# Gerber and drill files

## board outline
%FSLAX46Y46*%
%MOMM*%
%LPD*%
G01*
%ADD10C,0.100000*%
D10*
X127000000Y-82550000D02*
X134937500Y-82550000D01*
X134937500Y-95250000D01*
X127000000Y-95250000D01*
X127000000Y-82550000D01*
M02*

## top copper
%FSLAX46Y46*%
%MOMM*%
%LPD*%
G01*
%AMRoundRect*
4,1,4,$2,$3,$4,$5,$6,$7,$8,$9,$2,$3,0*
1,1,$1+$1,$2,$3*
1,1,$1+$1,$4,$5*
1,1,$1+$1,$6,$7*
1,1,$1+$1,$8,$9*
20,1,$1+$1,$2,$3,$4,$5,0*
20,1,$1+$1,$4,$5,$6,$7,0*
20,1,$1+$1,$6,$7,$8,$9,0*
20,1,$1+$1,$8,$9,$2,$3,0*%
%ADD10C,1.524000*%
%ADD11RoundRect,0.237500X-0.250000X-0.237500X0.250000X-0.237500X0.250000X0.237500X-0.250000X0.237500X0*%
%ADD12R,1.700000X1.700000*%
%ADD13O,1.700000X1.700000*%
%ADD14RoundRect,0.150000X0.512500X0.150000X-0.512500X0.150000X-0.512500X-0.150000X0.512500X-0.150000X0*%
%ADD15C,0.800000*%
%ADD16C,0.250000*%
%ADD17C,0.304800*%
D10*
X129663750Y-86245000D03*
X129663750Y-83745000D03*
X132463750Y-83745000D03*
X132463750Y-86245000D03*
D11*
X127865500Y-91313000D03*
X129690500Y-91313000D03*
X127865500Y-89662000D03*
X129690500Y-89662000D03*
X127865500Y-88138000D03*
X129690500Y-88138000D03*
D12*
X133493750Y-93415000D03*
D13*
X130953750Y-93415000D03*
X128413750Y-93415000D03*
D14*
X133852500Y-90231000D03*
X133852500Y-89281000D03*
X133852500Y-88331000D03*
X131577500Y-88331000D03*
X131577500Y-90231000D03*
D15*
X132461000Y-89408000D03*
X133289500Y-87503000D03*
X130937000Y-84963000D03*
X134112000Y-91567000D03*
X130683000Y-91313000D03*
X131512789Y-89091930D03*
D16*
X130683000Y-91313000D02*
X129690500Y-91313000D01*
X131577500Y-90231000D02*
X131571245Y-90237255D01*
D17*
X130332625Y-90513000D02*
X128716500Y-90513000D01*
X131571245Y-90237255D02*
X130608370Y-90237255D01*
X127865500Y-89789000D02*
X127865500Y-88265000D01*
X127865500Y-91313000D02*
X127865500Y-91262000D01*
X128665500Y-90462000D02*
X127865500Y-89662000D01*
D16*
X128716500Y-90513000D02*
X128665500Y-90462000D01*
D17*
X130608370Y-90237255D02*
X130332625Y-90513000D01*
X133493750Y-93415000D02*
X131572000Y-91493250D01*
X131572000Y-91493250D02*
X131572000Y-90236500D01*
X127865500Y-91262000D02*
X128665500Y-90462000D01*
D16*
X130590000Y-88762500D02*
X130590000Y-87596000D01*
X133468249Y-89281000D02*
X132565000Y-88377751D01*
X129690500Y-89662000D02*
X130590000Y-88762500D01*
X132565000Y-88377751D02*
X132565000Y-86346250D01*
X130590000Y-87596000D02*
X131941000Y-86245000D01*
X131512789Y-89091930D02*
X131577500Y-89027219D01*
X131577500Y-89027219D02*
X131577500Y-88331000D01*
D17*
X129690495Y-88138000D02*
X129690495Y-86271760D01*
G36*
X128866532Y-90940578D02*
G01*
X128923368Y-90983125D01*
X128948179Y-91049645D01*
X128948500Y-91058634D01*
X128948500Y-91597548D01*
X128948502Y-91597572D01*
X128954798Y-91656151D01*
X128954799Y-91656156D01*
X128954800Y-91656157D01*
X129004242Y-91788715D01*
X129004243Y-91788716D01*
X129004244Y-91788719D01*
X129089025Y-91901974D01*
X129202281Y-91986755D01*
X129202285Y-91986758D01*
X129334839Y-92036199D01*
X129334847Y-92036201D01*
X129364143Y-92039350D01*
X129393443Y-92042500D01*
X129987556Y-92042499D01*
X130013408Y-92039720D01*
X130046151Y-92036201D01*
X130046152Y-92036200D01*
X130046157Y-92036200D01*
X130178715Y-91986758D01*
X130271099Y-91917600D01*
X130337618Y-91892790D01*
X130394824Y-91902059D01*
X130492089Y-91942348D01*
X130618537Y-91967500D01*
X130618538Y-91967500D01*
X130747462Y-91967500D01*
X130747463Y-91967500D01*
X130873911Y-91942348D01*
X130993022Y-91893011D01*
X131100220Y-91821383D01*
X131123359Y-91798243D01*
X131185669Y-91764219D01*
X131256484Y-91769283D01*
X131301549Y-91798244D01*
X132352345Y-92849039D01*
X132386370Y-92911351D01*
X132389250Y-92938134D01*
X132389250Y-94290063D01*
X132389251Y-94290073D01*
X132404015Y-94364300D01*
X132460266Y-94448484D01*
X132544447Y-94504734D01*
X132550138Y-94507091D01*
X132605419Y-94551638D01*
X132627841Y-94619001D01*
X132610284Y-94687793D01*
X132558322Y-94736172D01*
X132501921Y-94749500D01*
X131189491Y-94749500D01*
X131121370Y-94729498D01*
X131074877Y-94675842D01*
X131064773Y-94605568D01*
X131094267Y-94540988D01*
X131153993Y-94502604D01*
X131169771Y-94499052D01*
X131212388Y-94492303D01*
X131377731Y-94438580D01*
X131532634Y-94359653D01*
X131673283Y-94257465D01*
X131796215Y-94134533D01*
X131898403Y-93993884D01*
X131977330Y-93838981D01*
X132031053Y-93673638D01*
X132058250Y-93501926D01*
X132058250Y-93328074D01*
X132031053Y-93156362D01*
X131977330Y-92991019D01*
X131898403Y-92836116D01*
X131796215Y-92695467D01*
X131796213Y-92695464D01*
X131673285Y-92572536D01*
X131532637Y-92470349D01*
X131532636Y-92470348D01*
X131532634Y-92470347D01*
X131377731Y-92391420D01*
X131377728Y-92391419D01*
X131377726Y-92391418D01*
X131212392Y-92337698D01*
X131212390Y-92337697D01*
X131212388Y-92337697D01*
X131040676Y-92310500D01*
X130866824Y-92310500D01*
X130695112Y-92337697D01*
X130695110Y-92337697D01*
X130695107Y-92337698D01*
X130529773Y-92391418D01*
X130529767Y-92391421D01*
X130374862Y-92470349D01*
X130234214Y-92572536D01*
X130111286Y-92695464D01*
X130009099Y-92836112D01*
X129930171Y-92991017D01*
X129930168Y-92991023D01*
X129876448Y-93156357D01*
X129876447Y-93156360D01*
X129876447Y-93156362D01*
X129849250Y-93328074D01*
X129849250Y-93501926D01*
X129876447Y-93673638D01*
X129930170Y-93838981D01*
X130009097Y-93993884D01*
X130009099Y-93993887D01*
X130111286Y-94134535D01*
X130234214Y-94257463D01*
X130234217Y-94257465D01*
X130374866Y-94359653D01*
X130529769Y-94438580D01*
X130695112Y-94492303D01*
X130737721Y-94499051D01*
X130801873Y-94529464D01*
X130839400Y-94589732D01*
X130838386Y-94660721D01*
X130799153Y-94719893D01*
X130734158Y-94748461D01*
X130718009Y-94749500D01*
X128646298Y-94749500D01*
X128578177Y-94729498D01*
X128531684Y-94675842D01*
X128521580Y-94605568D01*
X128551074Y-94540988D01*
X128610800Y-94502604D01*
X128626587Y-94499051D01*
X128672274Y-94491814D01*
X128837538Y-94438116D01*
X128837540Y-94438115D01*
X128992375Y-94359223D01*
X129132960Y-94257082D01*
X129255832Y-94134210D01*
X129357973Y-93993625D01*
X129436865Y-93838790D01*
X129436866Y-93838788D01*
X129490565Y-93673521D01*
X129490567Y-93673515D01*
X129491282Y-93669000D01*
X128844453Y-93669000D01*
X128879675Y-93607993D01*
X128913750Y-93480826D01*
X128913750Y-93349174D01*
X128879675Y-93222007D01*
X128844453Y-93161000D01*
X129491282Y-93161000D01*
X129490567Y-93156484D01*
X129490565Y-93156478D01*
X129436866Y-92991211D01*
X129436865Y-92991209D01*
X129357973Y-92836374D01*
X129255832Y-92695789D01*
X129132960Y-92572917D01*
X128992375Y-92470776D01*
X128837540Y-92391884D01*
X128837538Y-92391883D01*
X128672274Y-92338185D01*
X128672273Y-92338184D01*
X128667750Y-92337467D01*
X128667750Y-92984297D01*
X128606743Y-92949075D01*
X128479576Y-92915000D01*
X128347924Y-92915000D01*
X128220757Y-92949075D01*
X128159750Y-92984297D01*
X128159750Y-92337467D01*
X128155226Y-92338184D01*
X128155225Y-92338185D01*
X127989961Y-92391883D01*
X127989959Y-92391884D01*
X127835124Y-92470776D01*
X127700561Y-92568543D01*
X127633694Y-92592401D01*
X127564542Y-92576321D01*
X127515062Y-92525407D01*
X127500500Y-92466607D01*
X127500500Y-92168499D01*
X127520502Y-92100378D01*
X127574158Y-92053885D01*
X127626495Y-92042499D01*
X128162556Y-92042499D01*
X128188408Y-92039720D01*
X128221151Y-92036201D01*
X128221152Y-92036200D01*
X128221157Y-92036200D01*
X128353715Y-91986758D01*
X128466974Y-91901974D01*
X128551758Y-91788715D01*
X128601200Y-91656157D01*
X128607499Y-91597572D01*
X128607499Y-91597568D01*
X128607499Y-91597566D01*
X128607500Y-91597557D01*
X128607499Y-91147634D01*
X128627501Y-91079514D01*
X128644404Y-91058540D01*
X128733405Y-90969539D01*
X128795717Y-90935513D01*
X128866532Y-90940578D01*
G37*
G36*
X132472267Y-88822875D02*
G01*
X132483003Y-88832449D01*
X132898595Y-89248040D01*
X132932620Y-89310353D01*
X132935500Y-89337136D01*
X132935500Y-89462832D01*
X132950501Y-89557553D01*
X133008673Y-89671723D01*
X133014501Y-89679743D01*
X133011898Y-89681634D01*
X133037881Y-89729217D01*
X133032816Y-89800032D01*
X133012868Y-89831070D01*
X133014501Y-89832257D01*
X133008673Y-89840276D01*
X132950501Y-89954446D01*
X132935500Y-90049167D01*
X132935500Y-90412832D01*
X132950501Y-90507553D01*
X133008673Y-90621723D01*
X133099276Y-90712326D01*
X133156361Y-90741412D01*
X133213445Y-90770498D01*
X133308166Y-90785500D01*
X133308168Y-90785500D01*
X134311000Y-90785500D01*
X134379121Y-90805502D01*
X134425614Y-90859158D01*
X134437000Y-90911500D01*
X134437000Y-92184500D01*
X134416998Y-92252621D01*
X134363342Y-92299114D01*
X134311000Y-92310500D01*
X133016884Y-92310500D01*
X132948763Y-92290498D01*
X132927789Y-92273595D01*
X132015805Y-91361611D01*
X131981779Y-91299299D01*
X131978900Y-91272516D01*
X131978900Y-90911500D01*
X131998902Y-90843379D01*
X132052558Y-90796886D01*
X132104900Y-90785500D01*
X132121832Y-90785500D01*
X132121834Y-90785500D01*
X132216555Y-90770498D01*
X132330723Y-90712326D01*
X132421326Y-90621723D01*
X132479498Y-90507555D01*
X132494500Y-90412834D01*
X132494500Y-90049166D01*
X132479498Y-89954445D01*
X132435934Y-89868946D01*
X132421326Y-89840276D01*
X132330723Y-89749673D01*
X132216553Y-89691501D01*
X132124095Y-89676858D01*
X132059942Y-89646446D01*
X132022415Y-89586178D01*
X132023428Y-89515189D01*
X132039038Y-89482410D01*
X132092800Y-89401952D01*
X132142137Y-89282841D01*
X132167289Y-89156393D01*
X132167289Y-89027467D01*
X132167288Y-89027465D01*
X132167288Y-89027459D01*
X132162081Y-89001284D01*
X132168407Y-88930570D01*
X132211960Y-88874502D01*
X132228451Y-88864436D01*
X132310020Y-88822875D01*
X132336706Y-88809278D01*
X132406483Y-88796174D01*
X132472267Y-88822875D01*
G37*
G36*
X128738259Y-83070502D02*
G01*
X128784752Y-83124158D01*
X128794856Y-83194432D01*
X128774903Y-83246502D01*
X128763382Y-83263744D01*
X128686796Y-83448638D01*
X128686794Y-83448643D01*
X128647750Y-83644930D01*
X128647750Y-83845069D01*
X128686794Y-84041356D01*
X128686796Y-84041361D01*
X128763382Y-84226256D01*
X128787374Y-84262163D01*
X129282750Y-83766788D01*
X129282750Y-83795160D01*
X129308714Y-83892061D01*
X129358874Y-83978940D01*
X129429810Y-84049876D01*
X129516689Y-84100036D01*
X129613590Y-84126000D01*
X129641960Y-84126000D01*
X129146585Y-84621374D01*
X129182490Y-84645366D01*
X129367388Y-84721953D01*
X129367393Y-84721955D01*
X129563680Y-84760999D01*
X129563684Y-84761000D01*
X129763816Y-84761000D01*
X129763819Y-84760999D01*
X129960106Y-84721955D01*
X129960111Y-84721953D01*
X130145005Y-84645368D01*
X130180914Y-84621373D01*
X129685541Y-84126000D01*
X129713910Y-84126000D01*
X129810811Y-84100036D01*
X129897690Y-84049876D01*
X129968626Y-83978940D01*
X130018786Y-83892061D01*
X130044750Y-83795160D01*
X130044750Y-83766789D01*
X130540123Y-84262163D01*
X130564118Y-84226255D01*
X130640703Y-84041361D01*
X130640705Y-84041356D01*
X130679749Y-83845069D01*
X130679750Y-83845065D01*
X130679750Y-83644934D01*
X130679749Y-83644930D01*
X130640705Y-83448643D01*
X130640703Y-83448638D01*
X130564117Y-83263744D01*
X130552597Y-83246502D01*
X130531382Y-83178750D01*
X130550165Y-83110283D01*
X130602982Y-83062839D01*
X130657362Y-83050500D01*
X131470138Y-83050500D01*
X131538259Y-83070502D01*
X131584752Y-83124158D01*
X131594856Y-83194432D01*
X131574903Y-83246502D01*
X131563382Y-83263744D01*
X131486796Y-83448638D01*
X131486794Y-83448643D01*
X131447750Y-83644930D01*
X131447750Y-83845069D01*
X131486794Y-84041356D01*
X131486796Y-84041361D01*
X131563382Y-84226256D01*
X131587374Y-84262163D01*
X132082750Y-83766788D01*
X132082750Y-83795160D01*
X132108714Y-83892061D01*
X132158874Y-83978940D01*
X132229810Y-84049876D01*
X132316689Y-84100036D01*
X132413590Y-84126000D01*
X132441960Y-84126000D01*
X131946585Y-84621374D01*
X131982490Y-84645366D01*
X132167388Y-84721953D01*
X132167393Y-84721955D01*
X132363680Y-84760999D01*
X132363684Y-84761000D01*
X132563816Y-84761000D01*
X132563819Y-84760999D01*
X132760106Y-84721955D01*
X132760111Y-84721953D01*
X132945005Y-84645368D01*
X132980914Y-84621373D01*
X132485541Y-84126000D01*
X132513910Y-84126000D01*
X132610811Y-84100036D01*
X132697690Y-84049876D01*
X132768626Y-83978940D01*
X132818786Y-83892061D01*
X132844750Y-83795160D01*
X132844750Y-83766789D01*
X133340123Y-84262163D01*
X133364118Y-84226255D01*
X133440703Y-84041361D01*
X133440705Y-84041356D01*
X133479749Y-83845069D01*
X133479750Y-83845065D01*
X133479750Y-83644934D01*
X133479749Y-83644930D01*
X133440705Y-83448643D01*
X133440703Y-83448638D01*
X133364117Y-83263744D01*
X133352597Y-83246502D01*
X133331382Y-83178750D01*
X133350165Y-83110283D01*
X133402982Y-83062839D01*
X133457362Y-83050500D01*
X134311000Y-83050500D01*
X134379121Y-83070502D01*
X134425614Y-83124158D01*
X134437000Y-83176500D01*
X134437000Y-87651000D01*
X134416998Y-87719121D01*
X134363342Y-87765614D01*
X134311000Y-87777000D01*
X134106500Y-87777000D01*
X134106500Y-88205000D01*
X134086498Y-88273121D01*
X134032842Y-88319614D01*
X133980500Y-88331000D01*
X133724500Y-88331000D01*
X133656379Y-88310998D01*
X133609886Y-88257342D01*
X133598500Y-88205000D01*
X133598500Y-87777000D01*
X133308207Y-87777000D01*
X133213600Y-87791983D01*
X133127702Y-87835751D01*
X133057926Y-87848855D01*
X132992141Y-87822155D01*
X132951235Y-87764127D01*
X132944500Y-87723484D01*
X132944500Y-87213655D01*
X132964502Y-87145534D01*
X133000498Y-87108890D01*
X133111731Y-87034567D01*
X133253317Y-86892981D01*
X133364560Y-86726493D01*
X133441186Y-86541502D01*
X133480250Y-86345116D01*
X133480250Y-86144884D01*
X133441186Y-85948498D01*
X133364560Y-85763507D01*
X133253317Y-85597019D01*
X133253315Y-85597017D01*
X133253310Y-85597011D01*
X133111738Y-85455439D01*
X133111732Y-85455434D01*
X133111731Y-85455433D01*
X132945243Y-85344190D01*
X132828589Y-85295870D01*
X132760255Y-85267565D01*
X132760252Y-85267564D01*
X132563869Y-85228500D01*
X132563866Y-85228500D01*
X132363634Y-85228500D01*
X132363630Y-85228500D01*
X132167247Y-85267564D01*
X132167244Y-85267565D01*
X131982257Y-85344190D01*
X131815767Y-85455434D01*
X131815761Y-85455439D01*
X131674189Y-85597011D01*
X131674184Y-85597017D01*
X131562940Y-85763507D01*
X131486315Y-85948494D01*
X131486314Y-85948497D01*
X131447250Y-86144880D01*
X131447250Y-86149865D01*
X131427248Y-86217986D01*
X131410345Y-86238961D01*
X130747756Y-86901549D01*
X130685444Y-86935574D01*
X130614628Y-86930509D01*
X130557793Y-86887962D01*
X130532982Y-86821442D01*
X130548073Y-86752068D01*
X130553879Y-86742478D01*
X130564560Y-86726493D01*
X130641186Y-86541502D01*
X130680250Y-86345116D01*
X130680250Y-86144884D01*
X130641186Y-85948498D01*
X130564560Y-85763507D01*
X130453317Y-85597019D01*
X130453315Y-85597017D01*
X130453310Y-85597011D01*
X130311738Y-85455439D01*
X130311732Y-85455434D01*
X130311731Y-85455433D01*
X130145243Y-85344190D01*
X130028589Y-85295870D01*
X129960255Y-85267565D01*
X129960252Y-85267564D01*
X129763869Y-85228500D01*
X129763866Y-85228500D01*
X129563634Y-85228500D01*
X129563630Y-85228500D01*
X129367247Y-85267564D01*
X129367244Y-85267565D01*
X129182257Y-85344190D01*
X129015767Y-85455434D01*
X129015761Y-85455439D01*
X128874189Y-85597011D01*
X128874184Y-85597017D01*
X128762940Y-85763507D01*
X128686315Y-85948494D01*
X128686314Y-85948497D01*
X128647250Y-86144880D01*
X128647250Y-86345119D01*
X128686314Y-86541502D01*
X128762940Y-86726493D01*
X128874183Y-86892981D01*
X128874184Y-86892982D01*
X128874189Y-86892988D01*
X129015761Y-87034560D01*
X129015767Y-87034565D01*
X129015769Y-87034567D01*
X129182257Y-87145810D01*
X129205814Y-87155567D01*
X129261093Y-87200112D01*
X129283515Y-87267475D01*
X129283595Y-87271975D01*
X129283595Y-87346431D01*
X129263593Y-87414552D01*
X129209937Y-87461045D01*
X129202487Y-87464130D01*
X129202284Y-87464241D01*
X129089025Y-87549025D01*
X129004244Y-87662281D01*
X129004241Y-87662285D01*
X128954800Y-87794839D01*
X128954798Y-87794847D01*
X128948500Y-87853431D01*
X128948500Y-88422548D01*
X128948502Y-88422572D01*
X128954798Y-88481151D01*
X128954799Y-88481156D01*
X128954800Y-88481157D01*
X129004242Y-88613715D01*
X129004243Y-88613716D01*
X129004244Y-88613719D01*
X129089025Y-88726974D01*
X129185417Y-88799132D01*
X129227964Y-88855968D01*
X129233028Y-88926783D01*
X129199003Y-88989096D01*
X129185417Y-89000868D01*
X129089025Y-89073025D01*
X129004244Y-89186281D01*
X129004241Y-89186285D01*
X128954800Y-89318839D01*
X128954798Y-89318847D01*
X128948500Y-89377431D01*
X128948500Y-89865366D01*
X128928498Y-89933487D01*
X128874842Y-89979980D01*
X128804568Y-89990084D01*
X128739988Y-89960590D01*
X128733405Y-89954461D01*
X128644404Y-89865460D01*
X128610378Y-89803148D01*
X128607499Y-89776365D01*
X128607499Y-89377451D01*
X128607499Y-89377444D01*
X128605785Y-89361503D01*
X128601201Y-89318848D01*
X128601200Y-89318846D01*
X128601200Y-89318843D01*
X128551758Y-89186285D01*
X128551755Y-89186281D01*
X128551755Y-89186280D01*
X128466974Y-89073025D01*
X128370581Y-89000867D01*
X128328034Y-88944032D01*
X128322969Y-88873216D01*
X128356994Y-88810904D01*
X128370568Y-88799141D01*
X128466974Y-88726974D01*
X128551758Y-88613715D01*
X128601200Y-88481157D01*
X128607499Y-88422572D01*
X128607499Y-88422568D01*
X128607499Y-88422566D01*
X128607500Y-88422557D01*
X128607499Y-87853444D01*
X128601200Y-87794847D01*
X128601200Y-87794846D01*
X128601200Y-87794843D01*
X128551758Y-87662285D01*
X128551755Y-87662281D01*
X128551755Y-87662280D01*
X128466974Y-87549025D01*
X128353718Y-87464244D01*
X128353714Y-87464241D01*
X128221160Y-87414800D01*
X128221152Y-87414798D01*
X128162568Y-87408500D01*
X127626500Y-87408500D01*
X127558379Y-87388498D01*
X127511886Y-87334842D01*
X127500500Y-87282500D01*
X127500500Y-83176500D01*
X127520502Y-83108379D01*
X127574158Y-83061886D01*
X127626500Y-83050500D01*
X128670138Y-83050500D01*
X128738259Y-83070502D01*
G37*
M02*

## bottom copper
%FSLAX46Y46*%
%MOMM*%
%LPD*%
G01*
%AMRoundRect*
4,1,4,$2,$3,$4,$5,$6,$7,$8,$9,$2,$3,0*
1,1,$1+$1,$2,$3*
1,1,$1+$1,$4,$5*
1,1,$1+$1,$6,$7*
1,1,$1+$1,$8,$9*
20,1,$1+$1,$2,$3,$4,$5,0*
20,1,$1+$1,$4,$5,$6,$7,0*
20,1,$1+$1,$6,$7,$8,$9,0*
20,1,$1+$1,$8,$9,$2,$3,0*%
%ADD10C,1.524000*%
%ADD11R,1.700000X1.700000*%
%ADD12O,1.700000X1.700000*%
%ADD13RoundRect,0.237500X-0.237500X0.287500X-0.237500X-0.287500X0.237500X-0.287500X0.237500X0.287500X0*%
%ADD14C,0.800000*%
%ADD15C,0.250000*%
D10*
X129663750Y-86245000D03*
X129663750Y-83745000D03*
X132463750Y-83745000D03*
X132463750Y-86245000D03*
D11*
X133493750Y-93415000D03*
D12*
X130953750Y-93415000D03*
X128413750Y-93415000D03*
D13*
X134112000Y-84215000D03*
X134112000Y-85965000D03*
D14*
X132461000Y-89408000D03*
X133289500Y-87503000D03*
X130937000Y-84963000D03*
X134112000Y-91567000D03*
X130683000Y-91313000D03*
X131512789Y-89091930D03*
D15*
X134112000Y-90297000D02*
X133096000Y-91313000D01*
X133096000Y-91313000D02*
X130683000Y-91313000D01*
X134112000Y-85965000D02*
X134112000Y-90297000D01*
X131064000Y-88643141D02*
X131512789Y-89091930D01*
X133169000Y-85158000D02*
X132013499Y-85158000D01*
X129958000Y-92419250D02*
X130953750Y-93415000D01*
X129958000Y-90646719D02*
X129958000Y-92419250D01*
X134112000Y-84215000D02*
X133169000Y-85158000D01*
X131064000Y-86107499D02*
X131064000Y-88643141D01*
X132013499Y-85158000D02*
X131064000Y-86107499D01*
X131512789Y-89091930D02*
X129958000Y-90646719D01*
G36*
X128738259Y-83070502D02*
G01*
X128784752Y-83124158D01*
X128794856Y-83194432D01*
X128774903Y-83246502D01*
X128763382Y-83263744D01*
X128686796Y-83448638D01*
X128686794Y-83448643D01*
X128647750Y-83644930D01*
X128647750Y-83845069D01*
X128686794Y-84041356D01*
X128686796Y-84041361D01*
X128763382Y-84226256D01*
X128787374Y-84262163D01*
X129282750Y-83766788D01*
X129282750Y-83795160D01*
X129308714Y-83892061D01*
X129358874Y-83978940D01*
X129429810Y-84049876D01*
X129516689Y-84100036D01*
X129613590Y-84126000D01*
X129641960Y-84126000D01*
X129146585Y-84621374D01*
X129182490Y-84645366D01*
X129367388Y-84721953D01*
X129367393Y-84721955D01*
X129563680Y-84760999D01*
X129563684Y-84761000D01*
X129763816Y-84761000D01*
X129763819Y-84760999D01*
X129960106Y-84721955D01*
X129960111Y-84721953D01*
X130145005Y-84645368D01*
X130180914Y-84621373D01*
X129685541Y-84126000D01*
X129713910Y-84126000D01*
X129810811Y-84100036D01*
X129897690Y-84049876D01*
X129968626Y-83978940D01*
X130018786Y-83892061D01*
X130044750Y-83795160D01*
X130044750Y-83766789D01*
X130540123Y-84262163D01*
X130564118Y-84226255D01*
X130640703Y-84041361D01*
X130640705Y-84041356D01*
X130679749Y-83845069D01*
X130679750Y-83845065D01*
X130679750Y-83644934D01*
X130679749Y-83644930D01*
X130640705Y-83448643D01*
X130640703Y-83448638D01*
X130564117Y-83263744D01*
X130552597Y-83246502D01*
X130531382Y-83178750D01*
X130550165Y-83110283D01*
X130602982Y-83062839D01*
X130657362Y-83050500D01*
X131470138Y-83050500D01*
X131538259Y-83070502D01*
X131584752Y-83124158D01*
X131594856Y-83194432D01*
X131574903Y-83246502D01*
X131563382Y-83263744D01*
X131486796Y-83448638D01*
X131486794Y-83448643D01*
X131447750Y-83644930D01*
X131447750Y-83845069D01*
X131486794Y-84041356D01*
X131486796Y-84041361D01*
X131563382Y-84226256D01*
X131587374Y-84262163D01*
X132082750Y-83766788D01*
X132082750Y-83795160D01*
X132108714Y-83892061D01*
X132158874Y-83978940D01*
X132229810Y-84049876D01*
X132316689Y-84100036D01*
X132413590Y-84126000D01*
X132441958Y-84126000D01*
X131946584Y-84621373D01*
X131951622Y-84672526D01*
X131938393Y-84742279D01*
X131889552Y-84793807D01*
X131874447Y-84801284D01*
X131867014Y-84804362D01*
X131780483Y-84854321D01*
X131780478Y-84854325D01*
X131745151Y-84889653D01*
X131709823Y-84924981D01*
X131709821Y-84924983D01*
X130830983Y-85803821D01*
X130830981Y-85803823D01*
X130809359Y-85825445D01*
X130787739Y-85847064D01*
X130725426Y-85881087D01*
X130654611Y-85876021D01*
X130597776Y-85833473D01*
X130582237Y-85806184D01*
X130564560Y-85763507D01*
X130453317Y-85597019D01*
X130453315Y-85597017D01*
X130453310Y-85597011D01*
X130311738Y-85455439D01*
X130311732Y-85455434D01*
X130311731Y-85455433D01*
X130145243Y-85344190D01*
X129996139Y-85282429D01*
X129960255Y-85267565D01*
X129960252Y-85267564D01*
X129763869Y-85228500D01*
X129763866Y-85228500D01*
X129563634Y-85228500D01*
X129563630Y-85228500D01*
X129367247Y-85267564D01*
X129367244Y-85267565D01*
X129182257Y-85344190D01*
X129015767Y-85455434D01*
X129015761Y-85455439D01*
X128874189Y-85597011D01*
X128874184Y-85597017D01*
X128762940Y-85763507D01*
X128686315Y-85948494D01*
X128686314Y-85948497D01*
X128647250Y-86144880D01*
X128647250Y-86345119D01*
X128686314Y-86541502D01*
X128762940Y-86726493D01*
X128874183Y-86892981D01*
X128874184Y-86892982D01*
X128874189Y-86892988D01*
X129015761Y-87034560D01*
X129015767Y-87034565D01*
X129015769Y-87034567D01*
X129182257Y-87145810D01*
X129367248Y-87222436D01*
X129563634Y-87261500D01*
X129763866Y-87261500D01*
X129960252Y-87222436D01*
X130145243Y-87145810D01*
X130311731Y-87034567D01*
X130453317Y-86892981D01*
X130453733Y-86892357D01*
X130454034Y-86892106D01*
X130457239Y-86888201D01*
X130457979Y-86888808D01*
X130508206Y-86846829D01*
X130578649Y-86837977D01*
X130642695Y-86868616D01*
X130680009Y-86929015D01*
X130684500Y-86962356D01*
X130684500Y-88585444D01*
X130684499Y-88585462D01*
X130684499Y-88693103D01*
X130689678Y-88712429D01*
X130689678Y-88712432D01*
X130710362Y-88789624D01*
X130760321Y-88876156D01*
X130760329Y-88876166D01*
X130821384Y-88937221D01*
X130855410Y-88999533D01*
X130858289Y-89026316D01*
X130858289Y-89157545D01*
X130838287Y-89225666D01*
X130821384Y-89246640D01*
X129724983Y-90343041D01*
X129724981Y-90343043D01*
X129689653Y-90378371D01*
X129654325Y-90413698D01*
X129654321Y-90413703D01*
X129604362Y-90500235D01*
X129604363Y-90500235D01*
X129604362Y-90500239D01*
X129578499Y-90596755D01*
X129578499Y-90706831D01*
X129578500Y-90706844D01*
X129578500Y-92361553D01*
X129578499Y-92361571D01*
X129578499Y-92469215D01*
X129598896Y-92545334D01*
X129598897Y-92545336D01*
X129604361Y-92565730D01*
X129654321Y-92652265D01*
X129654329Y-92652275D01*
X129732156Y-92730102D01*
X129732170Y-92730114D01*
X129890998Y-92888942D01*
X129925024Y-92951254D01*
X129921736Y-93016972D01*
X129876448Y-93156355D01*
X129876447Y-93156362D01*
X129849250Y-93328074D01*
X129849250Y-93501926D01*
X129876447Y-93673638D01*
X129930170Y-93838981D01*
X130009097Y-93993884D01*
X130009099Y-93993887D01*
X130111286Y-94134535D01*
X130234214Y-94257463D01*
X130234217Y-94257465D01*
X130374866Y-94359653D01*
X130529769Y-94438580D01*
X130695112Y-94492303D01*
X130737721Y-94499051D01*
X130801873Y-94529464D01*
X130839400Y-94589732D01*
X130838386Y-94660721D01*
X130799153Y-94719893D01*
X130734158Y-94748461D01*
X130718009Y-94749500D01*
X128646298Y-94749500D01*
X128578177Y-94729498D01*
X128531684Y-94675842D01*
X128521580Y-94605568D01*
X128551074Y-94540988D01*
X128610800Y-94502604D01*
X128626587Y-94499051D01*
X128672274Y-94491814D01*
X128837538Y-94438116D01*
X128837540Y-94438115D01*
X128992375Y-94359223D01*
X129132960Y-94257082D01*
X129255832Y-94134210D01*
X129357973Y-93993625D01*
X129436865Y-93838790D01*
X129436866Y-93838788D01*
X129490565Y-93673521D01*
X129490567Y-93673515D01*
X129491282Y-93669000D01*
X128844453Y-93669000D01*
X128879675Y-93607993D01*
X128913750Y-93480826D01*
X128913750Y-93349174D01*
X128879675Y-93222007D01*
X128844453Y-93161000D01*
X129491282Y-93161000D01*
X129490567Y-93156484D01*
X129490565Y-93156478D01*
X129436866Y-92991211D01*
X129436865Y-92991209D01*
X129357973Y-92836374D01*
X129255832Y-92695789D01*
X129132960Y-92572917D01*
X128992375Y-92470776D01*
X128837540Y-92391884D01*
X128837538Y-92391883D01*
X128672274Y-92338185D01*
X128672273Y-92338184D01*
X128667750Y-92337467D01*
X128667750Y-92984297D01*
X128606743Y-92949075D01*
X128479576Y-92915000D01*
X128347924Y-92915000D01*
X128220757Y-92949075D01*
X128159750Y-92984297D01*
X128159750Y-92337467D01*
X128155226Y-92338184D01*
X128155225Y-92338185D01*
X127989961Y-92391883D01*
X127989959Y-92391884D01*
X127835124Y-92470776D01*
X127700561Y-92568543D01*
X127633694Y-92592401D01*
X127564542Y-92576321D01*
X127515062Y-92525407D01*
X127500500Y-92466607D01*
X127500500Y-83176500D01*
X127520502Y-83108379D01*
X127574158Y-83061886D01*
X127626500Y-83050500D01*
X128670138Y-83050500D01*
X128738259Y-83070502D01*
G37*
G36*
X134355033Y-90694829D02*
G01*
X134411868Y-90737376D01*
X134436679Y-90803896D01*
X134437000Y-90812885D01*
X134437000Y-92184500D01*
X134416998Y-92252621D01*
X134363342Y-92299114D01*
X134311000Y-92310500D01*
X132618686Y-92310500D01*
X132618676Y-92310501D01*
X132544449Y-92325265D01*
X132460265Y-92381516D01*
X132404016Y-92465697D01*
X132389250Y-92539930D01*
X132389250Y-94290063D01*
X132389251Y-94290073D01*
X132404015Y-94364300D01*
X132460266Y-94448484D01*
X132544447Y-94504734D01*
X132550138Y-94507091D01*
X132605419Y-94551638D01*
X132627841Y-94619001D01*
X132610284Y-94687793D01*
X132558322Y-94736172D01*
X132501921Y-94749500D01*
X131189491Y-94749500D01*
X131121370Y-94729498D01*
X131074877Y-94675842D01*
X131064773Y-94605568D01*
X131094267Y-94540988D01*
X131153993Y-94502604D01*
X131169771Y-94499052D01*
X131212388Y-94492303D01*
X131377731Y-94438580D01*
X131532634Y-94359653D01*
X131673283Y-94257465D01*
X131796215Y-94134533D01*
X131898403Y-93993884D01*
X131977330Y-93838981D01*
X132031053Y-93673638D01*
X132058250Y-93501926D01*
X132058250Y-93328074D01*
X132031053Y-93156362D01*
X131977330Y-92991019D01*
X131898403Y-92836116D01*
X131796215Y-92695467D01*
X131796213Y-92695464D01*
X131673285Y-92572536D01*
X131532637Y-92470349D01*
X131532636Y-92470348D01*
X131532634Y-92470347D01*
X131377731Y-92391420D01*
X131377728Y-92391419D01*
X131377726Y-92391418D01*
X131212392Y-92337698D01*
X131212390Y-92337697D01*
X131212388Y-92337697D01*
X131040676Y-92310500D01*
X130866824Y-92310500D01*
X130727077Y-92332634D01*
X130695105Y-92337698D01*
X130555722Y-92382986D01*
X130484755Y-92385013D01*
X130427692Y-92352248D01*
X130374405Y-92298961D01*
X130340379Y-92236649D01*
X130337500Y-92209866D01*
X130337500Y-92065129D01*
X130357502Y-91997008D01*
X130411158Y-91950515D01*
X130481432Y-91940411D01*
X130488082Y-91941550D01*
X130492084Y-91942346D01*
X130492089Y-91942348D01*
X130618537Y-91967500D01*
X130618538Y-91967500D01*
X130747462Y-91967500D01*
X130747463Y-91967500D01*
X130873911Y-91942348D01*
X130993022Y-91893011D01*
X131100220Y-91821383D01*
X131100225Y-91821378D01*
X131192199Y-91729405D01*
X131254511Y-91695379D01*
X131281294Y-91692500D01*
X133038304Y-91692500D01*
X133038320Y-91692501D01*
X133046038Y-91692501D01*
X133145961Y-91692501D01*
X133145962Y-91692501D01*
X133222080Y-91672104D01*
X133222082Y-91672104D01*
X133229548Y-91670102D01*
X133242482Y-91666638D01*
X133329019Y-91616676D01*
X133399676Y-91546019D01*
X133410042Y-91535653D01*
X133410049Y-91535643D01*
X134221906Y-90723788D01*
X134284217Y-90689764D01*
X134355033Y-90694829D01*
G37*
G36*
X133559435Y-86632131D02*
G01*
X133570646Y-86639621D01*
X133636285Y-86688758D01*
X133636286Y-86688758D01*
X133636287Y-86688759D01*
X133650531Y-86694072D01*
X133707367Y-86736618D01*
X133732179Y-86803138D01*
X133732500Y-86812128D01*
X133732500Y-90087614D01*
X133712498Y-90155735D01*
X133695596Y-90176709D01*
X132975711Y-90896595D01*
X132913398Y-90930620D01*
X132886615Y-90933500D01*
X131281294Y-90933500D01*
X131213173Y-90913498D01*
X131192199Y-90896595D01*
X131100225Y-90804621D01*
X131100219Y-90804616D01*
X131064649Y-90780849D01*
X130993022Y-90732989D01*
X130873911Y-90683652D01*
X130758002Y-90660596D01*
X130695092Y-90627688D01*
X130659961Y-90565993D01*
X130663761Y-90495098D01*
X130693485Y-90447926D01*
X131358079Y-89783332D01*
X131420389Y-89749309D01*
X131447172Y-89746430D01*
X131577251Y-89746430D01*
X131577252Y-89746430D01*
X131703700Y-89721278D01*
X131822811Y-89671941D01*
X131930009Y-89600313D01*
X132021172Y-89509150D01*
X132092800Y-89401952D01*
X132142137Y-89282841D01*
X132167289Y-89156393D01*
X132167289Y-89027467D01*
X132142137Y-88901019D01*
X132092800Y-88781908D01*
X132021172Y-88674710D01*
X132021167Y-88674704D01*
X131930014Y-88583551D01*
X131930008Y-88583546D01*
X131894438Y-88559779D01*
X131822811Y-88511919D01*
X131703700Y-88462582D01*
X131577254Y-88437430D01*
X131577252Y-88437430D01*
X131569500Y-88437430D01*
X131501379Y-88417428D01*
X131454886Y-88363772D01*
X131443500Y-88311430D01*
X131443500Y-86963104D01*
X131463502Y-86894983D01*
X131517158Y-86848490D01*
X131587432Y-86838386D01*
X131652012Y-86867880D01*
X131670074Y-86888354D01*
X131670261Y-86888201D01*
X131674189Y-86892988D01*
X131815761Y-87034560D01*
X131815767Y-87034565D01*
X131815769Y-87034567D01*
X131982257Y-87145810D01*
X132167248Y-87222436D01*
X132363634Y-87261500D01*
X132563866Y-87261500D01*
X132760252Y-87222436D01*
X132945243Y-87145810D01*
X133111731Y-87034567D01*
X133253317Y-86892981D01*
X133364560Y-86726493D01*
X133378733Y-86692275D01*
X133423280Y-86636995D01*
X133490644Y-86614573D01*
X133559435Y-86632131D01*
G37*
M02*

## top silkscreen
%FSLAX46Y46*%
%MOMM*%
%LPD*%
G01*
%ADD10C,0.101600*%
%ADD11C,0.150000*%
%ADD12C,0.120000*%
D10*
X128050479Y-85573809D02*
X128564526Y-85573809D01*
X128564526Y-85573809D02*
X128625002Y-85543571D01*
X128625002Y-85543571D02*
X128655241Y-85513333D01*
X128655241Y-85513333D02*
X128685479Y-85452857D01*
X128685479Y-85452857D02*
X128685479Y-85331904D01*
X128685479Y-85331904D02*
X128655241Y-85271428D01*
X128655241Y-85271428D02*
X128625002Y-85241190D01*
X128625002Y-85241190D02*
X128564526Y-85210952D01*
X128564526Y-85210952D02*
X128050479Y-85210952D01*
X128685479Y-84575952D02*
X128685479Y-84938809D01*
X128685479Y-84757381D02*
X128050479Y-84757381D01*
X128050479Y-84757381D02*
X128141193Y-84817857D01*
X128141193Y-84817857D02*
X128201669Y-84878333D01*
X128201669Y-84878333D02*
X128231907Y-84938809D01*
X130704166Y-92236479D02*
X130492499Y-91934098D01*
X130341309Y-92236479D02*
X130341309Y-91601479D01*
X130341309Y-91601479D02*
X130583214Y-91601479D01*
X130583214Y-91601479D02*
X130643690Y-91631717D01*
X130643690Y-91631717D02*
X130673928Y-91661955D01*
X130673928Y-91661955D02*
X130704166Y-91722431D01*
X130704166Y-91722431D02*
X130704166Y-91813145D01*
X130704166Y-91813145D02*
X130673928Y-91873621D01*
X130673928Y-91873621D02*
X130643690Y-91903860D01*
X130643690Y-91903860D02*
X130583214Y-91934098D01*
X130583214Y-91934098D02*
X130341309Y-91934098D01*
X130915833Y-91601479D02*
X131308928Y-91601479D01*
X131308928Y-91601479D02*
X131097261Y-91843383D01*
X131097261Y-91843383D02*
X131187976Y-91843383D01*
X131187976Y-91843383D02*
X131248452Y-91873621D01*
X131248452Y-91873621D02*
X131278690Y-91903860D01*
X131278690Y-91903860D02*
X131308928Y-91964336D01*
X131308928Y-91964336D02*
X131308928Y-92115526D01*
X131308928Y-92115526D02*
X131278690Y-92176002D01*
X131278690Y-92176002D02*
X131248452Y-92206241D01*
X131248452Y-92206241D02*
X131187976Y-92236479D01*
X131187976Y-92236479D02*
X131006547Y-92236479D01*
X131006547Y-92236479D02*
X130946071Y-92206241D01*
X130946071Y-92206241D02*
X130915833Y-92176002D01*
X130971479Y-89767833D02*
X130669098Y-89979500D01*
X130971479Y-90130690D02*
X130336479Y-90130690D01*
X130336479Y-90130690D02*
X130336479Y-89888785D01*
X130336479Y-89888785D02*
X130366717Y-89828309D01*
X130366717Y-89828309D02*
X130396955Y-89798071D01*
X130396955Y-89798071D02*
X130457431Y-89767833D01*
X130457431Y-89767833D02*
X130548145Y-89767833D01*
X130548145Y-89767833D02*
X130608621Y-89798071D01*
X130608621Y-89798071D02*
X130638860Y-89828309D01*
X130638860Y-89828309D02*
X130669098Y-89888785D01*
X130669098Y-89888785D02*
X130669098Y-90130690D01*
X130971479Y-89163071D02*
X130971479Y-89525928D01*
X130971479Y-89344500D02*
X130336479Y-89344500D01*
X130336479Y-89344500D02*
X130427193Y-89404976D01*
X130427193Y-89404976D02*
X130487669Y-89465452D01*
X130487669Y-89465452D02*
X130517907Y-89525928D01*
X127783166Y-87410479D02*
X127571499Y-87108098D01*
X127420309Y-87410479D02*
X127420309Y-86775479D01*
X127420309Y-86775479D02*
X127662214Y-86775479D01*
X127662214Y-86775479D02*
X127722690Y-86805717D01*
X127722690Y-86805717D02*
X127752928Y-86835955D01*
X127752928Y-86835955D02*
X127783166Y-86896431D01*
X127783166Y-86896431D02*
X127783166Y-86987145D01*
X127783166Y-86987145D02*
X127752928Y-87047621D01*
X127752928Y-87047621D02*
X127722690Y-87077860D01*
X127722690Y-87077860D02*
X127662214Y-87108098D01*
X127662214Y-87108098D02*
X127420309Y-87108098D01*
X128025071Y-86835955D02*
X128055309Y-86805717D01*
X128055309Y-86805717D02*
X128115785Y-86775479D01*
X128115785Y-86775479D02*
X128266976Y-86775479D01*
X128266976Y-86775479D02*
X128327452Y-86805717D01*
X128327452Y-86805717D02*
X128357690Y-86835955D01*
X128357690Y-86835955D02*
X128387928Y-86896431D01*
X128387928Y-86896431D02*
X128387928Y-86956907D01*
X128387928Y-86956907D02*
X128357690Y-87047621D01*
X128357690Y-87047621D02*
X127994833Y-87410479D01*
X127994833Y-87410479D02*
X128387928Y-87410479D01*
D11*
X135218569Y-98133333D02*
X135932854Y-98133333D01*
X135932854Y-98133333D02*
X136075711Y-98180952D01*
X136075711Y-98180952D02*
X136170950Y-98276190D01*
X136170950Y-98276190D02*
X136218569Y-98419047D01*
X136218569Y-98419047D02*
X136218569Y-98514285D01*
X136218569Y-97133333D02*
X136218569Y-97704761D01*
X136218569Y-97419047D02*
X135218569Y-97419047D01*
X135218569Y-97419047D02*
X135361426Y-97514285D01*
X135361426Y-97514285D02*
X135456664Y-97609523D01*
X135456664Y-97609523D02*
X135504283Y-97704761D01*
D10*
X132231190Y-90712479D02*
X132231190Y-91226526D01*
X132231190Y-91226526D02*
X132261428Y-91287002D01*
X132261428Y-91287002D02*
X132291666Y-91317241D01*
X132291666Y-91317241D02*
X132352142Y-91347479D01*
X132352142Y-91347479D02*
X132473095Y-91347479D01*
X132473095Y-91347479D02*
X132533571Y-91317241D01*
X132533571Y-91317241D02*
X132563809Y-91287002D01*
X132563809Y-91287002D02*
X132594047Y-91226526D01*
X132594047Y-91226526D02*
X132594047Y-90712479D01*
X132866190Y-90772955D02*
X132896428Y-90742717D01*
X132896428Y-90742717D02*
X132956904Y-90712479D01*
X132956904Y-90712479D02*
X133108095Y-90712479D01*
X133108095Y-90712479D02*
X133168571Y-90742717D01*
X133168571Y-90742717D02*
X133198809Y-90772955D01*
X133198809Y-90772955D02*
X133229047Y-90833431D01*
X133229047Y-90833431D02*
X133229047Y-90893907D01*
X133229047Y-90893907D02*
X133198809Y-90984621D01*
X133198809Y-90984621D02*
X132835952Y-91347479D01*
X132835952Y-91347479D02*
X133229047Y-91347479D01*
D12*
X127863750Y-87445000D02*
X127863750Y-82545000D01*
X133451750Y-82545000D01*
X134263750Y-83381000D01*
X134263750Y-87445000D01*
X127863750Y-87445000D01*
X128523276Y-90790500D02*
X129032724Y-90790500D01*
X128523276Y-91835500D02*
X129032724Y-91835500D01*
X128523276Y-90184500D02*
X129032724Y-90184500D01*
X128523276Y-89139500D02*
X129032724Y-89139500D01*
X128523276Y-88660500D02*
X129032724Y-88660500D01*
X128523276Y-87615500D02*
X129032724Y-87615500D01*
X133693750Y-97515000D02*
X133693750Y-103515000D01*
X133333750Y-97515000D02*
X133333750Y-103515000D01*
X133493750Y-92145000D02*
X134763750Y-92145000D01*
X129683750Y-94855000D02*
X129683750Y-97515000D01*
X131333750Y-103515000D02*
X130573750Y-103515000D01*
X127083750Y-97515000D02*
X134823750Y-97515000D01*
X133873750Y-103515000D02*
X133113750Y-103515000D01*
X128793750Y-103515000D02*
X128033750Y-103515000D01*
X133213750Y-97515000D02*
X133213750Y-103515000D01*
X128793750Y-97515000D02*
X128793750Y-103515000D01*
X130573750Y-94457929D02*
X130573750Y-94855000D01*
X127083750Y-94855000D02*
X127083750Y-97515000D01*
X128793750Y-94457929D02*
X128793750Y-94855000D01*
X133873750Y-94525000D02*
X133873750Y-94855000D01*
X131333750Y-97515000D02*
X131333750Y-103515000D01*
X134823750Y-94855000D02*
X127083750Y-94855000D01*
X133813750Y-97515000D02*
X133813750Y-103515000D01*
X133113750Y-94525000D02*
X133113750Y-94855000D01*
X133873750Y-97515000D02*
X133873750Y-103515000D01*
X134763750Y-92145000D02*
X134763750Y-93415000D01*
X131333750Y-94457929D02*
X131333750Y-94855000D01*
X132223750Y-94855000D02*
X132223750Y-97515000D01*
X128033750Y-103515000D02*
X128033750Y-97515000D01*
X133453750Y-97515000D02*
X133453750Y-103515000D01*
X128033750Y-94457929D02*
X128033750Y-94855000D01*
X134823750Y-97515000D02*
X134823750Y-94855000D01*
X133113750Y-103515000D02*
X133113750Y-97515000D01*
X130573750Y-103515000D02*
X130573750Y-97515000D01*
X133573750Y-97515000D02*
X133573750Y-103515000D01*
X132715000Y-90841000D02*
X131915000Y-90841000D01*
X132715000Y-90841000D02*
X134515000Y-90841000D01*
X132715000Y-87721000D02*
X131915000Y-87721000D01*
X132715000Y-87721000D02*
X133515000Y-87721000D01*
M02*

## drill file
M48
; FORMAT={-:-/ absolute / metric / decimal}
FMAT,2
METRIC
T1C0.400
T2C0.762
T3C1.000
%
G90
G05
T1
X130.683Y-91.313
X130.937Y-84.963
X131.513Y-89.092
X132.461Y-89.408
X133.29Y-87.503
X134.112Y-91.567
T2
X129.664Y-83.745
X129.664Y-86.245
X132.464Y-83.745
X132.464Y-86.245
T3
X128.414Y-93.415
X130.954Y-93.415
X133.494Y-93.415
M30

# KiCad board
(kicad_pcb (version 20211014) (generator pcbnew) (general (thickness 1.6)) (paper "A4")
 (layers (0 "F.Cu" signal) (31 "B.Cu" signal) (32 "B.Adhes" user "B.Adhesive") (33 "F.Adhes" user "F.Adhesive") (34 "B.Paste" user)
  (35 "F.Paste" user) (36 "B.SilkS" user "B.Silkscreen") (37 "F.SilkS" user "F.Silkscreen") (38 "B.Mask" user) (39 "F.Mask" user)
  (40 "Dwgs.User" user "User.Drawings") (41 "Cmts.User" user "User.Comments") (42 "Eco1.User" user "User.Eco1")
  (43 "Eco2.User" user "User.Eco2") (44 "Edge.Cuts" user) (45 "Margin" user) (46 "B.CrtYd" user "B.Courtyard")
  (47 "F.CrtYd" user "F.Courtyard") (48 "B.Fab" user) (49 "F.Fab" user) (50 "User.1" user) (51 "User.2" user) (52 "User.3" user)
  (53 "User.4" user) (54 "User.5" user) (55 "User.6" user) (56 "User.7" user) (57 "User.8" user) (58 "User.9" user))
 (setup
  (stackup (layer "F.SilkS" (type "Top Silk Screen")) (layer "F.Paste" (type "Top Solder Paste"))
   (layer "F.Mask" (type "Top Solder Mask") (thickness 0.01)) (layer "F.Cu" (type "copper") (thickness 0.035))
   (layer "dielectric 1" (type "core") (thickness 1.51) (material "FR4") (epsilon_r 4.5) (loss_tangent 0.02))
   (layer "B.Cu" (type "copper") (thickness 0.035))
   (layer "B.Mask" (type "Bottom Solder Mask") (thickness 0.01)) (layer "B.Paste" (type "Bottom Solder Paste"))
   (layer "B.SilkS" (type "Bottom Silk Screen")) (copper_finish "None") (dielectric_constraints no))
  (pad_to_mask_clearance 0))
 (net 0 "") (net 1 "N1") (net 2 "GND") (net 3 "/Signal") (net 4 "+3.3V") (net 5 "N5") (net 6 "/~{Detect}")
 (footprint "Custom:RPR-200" (layer "F.Cu") (at 127.86375 87.445)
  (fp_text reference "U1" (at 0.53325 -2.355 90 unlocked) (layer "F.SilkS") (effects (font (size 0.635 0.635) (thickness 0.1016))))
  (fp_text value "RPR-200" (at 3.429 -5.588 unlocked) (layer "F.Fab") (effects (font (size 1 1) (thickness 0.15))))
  (fp_poly (pts (xy 0 0) (xy 0 -4.9) (xy 5.588 -4.9) (xy 6.4 -4.064) (xy 6.4 0)) (layer "F.SilkS") (width 0.12) (fill none))
  (pad "1" thru_hole circle (at 1.8 -1.2) (size 1.524 1.524) (drill 0.762) (layers *.Cu *.Mask) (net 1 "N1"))
  (pad "2" thru_hole circle (at 1.8 -3.7) (size 1.524 1.524) (drill 0.762) (layers *.Cu *.Mask) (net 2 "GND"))
  (pad "3" thru_hole circle (at 4.6 -3.7) (size 1.524 1.524) (drill 0.762) (layers *.Cu *.Mask) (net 2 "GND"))
  (pad "4" thru_hole circle (at 4.6 -1.2) (size 1.524 1.524) (drill 0.762) (layers *.Cu *.Mask) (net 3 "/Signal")))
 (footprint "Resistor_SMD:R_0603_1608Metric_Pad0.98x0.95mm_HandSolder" (layer "F.Cu") (at 128.778 91.313)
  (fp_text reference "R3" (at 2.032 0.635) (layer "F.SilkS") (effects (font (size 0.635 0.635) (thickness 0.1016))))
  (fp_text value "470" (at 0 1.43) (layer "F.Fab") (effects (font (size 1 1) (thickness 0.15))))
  (fp_line (start -0.254724 -0.5225) (end 0.254724 -0.5225) (layer "F.SilkS") (width 0.12))
  (fp_line (start -0.254724 0.5225) (end 0.254724 0.5225) (layer "F.SilkS") (width 0.12))
  (pad "1" smd roundrect (at -0.9125 0) (size 0.975 0.95) (layers "F.Cu" "F.Paste" "F.Mask") (roundrect_rratio 0.25) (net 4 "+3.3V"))
  (pad "2" smd roundrect (at 0.9125 0) (size 0.975 0.95) (layers "F.Cu" "F.Paste" "F.Mask") (roundrect_rratio 0.25) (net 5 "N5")))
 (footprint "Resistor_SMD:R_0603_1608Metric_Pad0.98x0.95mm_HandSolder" (layer "F.Cu") (at 128.778 89.662)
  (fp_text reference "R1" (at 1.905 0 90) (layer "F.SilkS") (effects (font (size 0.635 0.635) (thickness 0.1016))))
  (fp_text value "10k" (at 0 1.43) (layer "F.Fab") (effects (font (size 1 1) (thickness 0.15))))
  (fp_line (start -0.254724 0.5225) (end 0.254724 0.5225) (layer "F.SilkS") (width 0.12))
  (fp_line (start -0.254724 -0.5225) (end 0.254724 -0.5225) (layer "F.SilkS") (width 0.12))
  (pad "1" smd roundrect (at -0.9125 0) (size 0.975 0.95) (layers "F.Cu" "F.Paste" "F.Mask") (roundrect_rratio 0.25) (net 4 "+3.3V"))
  (pad "2" smd roundrect (at 0.9125 0) (size 0.975 0.95) (layers "F.Cu" "F.Paste" "F.Mask") (roundrect_rratio 0.25) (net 3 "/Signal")))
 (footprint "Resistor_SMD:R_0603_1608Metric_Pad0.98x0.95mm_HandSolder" (layer "F.Cu") (at 128.778 88.138)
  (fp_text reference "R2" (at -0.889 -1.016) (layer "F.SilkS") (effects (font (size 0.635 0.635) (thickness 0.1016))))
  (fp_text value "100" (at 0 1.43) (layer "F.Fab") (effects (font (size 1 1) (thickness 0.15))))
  (fp_line (start -0.254724 0.5225) (end 0.254724 0.5225) (layer "F.SilkS") (width 0.12))
  (fp_line (start -0.254724 -0.5225) (end 0.254724 -0.5225) (layer "F.SilkS") (width 0.12))
  (pad "1" smd roundrect (at -0.9125 0) (size 0.975 0.95) (layers "F.Cu" "F.Paste" "F.Mask") (roundrect_rratio 0.25) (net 4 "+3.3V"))
  (pad "2" smd roundrect (at 0.9125 0) (size 0.975 0.95) (layers "F.Cu" "F.Paste" "F.Mask") (roundrect_rratio 0.25) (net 1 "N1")))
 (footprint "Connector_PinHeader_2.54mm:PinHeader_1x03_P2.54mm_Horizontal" (layer "F.Cu") (at 133.49375 93.415 -90)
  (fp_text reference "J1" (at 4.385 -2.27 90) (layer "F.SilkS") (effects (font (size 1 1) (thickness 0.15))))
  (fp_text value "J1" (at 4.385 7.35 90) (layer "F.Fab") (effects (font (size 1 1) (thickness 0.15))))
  (fp_line (start 4.1 -0.2) (end 10.1 -0.2) (layer "F.SilkS") (width 0.12))
  (fp_line (start 4.1 0.16) (end 10.1 0.16) (layer "F.SilkS") (width 0.12))
  (fp_line (start -1.27 0) (end -1.27 -1.27) (layer "F.SilkS") (width 0.12))
  (fp_line (start 1.44 3.81) (end 4.1 3.81) (layer "F.SilkS") (width 0.12))
  (fp_line (start 10.1 2.16) (end 10.1 2.92) (layer "F.SilkS") (width 0.12))
  (fp_line (start 4.1 6.41) (end 4.1 -1.33) (layer "F.SilkS") (width 0.12))
  (fp_line (start 10.1 -0.38) (end 10.1 0.38) (layer "F.SilkS") (width 0.12))
  (fp_line (start 10.1 4.7) (end 10.1 5.46) (layer "F.SilkS") (width 0.12))
  (fp_line (start 4.1 0.28) (end 10.1 0.28) (layer "F.SilkS") (width 0.12))
  (fp_line (start 4.1 4.7) (end 10.1 4.7) (layer "F.SilkS") (width 0.12))
  (fp_line (start 1.042929 2.92) (end 1.44 2.92) (layer "F.SilkS") (width 0.12))
  (fp_line (start 1.44 6.41) (end 4.1 6.41) (layer "F.SilkS") (width 0.12))
  (fp_line (start 1.042929 4.7) (end 1.44 4.7) (layer "F.SilkS") (width 0.12))
  (fp_line (start 1.11 -0.38) (end 1.44 -0.38) (layer "F.SilkS") (width 0.12))
  (fp_line (start 4.1 2.16) (end 10.1 2.16) (layer "F.SilkS") (width 0.12))
  (fp_line (start 1.44 -1.33) (end 1.44 6.41) (layer "F.SilkS") (width 0.12))
  (fp_line (start 4.1 -0.32) (end 10.1 -0.32) (layer "F.SilkS") (width 0.12))
  (fp_line (start 1.11 0.38) (end 1.44 0.38) (layer "F.SilkS") (width 0.12))
  (fp_line (start 4.1 -0.38) (end 10.1 -0.38) (layer "F.SilkS") (width 0.12))
  (fp_line (start -1.27 -1.27) (end 0 -1.27) (layer "F.SilkS") (width 0.12))
  (fp_line (start 1.042929 2.16) (end 1.44 2.16) (layer "F.SilkS") (width 0.12))
  (fp_line (start 1.44 1.27) (end 4.1 1.27) (layer "F.SilkS") (width 0.12))
  (fp_line (start 10.1 5.46) (end 4.1 5.46) (layer "F.SilkS") (width 0.12))
  (fp_line (start 4.1 0.04) (end 10.1 0.04) (layer "F.SilkS") (width 0.12))
  (fp_line (start 1.042929 5.46) (end 1.44 5.46) (layer "F.SilkS") (width 0.12))
  (fp_line (start 4.1 -1.33) (end 1.44 -1.33) (layer "F.SilkS") (width 0.12))
  (fp_line (start 10.1 0.38) (end 4.1 0.38) (layer "F.SilkS") (width 0.12))
  (fp_line (start 10.1 2.92) (end 4.1 2.92) (layer "F.SilkS") (width 0.12))
  (fp_line (start 4.1 -0.08) (end 10.1 -0.08) (layer "F.SilkS") (width 0.12))
  (pad "1" thru_hole rect (at 0 0 270) (size 1.7 1.7) (drill 1) (layers *.Cu *.Mask) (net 4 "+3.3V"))
  (pad "2" thru_hole oval (at 0 2.54 270) (size 1.7 1.7) (drill 1) (layers *.Cu *.Mask) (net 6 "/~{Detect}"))
  (pad "3" thru_hole oval (at 0 5.08 270) (size 1.7 1.7) (drill 1) (layers *.Cu *.Mask) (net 2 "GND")))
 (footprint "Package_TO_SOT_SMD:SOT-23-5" (layer "F.Cu") (at 132.715 89.281 180)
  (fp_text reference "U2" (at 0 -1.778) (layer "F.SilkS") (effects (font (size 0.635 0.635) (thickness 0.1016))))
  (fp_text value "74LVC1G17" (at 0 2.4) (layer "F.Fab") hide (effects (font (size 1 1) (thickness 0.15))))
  (fp_line (start 0 -1.56) (end 0.8 -1.56) (layer "F.SilkS") (width 0.12))
  (fp_line (start 0 -1.56) (end -1.8 -1.56) (layer "F.SilkS") (width 0.12))
  (fp_line (start 0 1.56) (end 0.8 1.56) (layer "F.SilkS") (width 0.12))
  (fp_line (start 0 1.56) (end -0.8 1.56) (layer "F.SilkS") (width 0.12))
  (pad "1" smd roundrect (at -1.1375 -0.95 180) (size 1.325 0.6) (layers "F.Cu" "F.Paste" "F.Mask") (roundrect_rratio 0.25))
  (pad "2" smd roundrect (at -1.1375 0 180) (size 1.325 0.6) (layers "F.Cu" "F.Paste" "F.Mask") (roundrect_rratio 0.25) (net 3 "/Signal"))
  (pad "3" smd roundrect (at -1.1375 0.95 180) (size 1.325 0.6) (layers "F.Cu" "F.Paste" "F.Mask") (roundrect_rratio 0.25) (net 2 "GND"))
  (pad "4" smd roundrect (at 1.1375 0.95 180) (size 1.325 0.6) (layers "F.Cu" "F.Paste" "F.Mask") (roundrect_rratio 0.25)
   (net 6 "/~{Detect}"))
  (pad "5" smd roundrect (at 1.1375 -0.95 180) (size 1.325 0.6) (layers "F.Cu" "F.Paste" "F.Mask") (roundrect_rratio 0.25) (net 4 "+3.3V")))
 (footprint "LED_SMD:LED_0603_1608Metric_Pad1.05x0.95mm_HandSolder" (layer "B.Cu") (at 134.112 85.09 -90)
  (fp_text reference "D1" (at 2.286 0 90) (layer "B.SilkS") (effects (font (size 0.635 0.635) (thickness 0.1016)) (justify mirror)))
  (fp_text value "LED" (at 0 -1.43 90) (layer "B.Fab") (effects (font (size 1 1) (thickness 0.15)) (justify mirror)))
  (pad "1" smd roundrect (at -0.875 0 270) (size 1.05 0.95) (layers "B.Cu" "B.Paste" "B.Mask") (roundrect_rratio 0.25) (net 6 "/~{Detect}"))
  (pad "2" smd roundrect (at 0.875 0 270) (size 1.05 0.95) (layers "B.Cu" "B.Paste" "B.Mask") (roundrect_rratio 0.25) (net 5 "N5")))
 (gr_rect (start 127 82.55) (end 134.9375 95.25) (layer "Edge.Cuts") (width 0.1) (fill none))
 (via (at 132.461 89.408) (size 0.8) (drill 0.4) (layers "F.Cu" "B.Cu") (free) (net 2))
 (via (at 133.2895 87.503) (size 0.8) (drill 0.4) (layers "F.Cu" "B.Cu") (free) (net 2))
 (via (at 130.937 84.963) (size 0.8) (drill 0.4) (layers "F.Cu" "B.Cu") (free) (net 2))
 (via (at 134.112 91.567) (size 0.8) (drill 0.4) (layers "F.Cu" "B.Cu") (free) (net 2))
 (segment (start 130.683 91.313) (end 129.6905 91.313) (width 0.25) (layer "F.Cu") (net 5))
 (via (at 130.683 91.313) (size 0.8) (drill 0.4) (layers "F.Cu" "B.Cu") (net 5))
 (segment (start 134.112 90.297) (end 133.096 91.313) (width 0.25) (layer "B.Cu") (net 5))
 (segment (start 133.096 91.313) (end 130.683 91.313) (width 0.25) (layer "B.Cu") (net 5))
 (segment (start 134.112 85.965) (end 134.112 90.297) (width 0.25) (layer "B.Cu") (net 5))
 (segment (start 131.5775 90.231) (end 131.571245 90.237255) (width 0.25) (layer "F.Cu") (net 4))
 (segment (start 130.332625 90.513) (end 128.7165 90.513) (width 0.3048) (layer "F.Cu") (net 4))
 (segment (start 131.571245 90.237255) (end 130.60837 90.237255) (width 0.3048) (layer "F.Cu") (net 4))
 (segment (start 127.8655 89.789) (end 127.8655 88.265) (width 0.3048) (layer "F.Cu") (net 4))
 (segment (start 127.8655 91.313) (end 127.8655 91.262) (width 0.3048) (layer "F.Cu") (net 4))
 (segment (start 128.6655 90.462) (end 127.8655 89.662) (width 0.3048) (layer "F.Cu") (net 4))
 (segment (start 128.7165 90.513) (end 128.6655 90.462) (width 0.25) (layer "F.Cu") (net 4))
 (segment (start 130.60837 90.237255) (end 130.332625 90.513) (width 0.3048) (layer "F.Cu") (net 4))
 (segment (start 133.49375 93.415) (end 131.572 91.49325) (width 0.3048) (layer "F.Cu") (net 4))
 (segment (start 131.572 91.49325) (end 131.572 90.2365) (width 0.3048) (layer "F.Cu") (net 4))
 (segment (start 127.8655 91.262) (end 128.6655 90.462) (width 0.3048) (layer "F.Cu") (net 4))
 (segment (start 130.59 88.7625) (end 130.59 87.596) (width 0.25) (layer "F.Cu") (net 3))
 (segment (start 133.468249 89.281) (end 132.565 88.377751) (width 0.25) (layer "F.Cu") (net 3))
 (segment (start 129.6905 89.662) (end 130.59 88.7625) (width 0.25) (layer "F.Cu") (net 3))
 (segment (start 132.565 88.377751) (end 132.565 86.34625) (width 0.25) (layer "F.Cu") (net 3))
 (segment (start 130.59 87.596) (end 131.941 86.245) (width 0.25) (layer "F.Cu") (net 3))
 (segment (start 131.512789 89.09193) (end 131.5775 89.027219) (width 0.25) (layer "F.Cu") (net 6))
 (segment (start 131.5775 89.027219) (end 131.5775 88.331) (width 0.25) (layer "F.Cu") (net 6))
 (via (at 131.512789 89.09193) (size 0.8) (drill 0.4) (layers "F.Cu" "B.Cu") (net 6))
 (segment (start 131.064 88.643141) (end 131.512789 89.09193) (width 0.25) (layer "B.Cu") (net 6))
 (segment (start 133.169 85.158) (end 132.013499 85.158) (width 0.25) (layer "B.Cu") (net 6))
 (segment (start 129.958 92.41925) (end 130.95375 93.415) (width 0.25) (layer "B.Cu") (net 6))
 (segment (start 129.958 90.646719) (end 129.958 92.41925) (width 0.25) (layer "B.Cu") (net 6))
 (segment (start 134.112 84.215) (end 133.169 85.158) (width 0.25) (layer "B.Cu") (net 6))
 (segment (start 131.064 86.107499) (end 131.064 88.643141) (width 0.25) (layer "B.Cu") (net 6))
 (segment (start 132.013499 85.158) (end 131.064 86.107499) (width 0.25) (layer "B.Cu") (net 6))
 (segment (start 131.512789 89.09193) (end 129.958 90.646719) (width 0.25) (layer "B.Cu") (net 6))
 (segment (start 129.690495 88.138) (end 129.690495 86.27176) (width 0.3048) (layer "F.Cu") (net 1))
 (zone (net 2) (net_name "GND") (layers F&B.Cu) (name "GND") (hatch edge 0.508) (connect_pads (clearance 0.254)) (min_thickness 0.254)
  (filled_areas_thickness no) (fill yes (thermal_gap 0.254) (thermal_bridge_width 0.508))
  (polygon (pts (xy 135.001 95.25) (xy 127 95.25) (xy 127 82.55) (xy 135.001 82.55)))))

